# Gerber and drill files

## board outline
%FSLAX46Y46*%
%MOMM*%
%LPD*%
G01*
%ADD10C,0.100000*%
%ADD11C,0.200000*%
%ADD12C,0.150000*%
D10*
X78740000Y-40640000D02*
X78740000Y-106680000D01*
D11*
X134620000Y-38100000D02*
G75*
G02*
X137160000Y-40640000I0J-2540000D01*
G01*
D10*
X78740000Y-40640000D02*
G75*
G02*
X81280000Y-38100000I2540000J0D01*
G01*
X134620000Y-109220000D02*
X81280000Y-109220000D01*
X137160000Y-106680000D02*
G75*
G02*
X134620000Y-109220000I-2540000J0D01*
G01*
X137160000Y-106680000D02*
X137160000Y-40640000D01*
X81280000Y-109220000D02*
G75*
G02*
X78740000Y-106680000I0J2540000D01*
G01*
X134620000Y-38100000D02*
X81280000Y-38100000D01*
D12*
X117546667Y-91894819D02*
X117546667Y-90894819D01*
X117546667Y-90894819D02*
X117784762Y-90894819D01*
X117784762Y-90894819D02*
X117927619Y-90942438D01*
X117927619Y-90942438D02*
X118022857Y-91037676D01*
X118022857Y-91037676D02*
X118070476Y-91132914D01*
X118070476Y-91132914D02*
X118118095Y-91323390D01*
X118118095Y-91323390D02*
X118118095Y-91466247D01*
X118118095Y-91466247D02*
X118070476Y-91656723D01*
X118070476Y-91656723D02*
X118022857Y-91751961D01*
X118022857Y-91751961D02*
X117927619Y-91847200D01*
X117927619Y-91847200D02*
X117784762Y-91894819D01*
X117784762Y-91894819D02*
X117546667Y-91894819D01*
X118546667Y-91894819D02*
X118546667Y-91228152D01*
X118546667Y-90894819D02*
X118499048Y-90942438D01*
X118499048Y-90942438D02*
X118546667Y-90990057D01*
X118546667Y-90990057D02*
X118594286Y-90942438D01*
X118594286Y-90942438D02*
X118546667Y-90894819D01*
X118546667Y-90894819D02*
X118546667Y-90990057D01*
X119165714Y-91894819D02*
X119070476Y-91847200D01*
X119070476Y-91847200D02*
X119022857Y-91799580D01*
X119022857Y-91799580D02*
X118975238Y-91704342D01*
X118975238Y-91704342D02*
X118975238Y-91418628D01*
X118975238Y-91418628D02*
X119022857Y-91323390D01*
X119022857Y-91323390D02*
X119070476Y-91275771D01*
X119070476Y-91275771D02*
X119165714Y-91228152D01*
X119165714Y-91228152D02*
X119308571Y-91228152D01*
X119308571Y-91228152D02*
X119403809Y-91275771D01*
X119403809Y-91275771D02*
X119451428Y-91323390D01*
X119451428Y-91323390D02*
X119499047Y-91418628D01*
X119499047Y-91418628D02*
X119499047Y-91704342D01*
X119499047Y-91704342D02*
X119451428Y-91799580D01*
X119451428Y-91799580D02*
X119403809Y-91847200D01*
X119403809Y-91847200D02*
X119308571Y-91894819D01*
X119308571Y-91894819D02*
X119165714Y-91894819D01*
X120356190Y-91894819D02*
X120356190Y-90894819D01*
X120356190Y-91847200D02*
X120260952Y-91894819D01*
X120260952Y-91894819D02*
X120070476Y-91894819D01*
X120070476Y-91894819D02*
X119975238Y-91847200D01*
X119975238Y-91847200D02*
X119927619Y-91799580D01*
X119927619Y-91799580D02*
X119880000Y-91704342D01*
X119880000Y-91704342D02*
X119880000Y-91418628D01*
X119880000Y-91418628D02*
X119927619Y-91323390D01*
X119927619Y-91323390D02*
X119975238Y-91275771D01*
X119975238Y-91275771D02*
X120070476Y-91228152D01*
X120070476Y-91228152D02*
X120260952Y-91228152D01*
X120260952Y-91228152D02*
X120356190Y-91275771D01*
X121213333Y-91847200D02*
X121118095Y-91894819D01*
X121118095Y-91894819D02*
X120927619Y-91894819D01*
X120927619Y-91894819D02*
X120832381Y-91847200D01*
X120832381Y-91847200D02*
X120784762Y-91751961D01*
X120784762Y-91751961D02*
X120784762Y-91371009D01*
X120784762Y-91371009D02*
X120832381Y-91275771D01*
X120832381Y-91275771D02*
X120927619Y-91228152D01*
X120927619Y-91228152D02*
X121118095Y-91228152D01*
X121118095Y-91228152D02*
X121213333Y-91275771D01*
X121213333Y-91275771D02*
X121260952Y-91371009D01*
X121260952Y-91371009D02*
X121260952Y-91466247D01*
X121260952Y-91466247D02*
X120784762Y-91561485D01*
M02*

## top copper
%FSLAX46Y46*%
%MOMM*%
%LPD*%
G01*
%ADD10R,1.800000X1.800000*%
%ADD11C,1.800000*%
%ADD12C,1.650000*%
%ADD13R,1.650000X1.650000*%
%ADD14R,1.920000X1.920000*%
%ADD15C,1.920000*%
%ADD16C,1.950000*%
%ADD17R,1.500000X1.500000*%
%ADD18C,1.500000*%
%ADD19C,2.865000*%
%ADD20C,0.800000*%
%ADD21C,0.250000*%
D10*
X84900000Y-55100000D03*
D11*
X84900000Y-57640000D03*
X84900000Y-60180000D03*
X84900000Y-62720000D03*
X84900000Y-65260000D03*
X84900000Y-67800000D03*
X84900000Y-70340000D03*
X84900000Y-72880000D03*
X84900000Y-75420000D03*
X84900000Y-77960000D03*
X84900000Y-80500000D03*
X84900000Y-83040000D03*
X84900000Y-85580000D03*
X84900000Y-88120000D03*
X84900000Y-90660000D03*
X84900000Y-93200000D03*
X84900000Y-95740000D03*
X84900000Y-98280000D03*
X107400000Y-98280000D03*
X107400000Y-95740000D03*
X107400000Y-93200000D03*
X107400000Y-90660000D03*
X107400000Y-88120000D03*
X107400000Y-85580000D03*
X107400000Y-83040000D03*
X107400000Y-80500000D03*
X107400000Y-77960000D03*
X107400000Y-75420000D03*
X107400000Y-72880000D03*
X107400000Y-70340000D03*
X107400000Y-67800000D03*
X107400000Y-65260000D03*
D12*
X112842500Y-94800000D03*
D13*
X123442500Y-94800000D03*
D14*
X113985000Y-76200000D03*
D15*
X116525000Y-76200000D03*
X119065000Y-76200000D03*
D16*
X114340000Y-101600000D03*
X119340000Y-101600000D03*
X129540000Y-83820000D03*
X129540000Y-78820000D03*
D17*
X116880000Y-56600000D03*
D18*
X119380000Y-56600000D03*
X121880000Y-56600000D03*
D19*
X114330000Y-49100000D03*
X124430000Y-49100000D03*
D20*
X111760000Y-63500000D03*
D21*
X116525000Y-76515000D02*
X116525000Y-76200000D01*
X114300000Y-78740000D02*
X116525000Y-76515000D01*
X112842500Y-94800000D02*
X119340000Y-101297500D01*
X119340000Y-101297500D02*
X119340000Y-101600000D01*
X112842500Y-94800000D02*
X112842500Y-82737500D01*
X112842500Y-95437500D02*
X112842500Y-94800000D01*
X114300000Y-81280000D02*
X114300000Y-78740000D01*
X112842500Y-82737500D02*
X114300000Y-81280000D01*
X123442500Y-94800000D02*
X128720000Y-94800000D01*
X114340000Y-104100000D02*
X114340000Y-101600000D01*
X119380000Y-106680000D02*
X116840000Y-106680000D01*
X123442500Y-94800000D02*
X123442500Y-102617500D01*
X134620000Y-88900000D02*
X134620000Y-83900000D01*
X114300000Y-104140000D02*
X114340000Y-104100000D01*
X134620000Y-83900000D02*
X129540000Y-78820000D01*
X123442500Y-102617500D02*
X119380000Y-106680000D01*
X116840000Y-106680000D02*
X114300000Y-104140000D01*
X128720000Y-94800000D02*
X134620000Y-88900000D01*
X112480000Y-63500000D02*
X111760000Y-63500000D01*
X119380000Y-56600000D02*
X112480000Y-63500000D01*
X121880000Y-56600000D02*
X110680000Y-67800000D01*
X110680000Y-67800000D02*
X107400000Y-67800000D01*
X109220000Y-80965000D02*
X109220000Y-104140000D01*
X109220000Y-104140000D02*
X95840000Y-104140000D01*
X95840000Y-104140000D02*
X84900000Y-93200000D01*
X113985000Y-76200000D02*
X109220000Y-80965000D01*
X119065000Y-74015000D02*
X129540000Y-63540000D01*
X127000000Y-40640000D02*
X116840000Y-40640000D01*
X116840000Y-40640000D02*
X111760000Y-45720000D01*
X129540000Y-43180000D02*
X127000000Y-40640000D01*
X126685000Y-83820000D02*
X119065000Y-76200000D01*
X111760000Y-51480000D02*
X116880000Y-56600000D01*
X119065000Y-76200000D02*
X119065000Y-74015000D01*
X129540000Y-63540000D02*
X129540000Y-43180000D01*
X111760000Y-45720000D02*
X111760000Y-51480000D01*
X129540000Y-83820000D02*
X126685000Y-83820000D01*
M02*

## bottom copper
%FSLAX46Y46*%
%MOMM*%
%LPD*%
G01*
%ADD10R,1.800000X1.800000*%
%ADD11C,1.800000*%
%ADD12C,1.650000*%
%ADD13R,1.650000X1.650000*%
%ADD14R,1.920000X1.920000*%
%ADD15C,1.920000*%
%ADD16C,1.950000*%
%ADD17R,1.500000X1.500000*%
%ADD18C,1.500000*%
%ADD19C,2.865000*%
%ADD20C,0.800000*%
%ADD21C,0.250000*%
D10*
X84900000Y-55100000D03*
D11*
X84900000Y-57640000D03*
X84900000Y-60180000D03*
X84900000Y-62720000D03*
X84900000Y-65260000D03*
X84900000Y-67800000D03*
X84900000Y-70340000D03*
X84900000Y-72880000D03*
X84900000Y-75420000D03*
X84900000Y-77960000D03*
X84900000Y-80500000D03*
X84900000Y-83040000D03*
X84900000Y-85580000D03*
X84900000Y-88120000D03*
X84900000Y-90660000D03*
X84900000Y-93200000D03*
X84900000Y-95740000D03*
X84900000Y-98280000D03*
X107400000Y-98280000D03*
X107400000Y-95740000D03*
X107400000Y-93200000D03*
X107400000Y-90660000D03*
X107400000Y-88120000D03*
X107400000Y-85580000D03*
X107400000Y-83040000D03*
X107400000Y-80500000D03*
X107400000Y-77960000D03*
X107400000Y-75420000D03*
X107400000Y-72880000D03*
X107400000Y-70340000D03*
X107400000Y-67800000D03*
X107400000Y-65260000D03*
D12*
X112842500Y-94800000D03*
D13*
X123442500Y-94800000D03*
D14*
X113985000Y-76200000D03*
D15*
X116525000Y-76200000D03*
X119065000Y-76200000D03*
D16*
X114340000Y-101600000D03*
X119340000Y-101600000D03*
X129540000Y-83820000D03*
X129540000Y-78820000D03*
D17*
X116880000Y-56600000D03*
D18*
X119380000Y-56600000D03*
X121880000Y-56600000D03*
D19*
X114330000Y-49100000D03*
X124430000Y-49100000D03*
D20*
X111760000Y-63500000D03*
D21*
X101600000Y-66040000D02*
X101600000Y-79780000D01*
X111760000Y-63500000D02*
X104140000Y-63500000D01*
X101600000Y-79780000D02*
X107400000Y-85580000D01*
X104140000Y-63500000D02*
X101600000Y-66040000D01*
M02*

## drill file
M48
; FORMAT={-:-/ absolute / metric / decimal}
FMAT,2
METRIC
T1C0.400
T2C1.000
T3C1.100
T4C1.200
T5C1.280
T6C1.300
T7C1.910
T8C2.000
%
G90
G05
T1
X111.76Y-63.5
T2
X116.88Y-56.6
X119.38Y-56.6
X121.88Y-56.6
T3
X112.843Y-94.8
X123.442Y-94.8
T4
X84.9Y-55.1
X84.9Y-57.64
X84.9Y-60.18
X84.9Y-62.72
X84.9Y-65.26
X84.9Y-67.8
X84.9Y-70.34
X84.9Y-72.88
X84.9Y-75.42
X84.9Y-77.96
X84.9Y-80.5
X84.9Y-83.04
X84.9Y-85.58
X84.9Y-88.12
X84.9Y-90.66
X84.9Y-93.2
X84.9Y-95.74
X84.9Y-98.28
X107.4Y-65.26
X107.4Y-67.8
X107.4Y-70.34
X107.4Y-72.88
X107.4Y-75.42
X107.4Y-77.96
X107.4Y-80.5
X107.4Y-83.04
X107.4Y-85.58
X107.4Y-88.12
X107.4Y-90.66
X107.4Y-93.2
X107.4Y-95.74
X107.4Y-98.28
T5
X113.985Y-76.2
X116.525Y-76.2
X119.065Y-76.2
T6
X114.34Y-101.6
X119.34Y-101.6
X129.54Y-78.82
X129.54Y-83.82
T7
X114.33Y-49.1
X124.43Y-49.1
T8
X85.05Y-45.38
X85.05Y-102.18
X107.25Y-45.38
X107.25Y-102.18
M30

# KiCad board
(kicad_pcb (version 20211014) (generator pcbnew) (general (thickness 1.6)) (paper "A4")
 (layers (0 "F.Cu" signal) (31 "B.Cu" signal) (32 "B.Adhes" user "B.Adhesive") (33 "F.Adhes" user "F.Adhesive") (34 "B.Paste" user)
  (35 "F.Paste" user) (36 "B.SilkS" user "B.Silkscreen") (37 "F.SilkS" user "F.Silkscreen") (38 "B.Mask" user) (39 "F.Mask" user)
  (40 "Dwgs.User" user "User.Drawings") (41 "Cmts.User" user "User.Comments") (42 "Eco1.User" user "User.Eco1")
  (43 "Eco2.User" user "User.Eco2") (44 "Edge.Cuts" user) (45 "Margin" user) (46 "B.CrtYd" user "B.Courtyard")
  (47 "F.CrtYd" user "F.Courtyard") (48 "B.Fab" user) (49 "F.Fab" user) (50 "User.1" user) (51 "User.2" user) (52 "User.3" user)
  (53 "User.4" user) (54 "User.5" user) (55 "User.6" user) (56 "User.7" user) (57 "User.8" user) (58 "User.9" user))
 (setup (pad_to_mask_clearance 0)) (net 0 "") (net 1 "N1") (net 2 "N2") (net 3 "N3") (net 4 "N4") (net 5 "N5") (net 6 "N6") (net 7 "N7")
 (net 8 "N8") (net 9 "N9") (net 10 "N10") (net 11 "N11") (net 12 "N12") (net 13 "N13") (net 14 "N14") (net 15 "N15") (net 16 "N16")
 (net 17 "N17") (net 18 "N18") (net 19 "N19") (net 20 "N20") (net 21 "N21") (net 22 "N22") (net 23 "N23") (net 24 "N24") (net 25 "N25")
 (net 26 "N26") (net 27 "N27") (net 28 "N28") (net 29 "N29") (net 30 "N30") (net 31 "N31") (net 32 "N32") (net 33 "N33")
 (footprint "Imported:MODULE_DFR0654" (layer "F.Cu") (at 96.15 73.78)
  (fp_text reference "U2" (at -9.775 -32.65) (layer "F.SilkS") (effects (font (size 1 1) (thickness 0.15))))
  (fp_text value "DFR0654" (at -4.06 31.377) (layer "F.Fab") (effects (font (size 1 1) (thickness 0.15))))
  (pad "" np_thru_hole circle (at 11.1 28.4) (size 2 2) (drill 2) (layers *.Cu *.Mask))
  (pad "" np_thru_hole circle (at 11.1 -28.4) (size 2 2) (drill 2) (layers *.Cu *.Mask))
  (pad "" np_thru_hole circle (at -11.1 -28.4) (size 2 2) (drill 2) (layers *.Cu *.Mask))
  (pad "" np_thru_hole circle (at -11.1 28.4) (size 2 2) (drill 2) (layers *.Cu *.Mask))
  (pad "1" thru_hole rect (at -11.25 -18.68) (size 1.8 1.8) (drill 1.2) (layers *.Cu *.Mask) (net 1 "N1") (solder_mask_margin 0.102))
  (pad "2" thru_hole circle (at -11.25 -16.14) (size 1.8 1.8) (drill 1.2) (layers *.Cu *.Mask) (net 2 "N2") (solder_mask_margin 0.102))
  (pad "3" thru_hole circle (at -11.25 -13.6) (size 1.8 1.8) (drill 1.2) (layers *.Cu *.Mask) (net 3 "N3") (solder_mask_margin 0.102))
  (pad "4" thru_hole circle (at -11.25 -11.06) (size 1.8 1.8) (drill 1.2) (layers *.Cu *.Mask) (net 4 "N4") (solder_mask_margin 0.102))
  (pad "5" thru_hole circle (at -11.25 -8.52) (size 1.8 1.8) (drill 1.2) (layers *.Cu *.Mask) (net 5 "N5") (solder_mask_margin 0.102))
  (pad "6" thru_hole circle (at -11.25 -5.98) (size 1.8 1.8) (drill 1.2) (layers *.Cu *.Mask) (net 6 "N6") (solder_mask_margin 0.102))
  (pad "7" thru_hole circle (at -11.25 -3.44) (size 1.8 1.8) (drill 1.2) (layers *.Cu *.Mask) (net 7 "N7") (solder_mask_margin 0.102))
  (pad "8" thru_hole circle (at -11.25 -0.9) (size 1.8 1.8) (drill 1.2) (layers *.Cu *.Mask) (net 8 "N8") (solder_mask_margin 0.102))
  (pad "9" thru_hole circle (at -11.25 1.64) (size 1.8 1.8) (drill 1.2) (layers *.Cu *.Mask) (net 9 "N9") (solder_mask_margin 0.102))
  (pad "10" thru_hole circle (at -11.25 4.18) (size 1.8 1.8) (drill 1.2) (layers *.Cu *.Mask) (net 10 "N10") (solder_mask_margin 0.102))
  (pad "11" thru_hole circle (at -11.25 6.72) (size 1.8 1.8) (drill 1.2) (layers *.Cu *.Mask) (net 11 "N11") (solder_mask_margin 0.102))
  (pad "12" thru_hole circle (at -11.25 9.26) (size 1.8 1.8) (drill 1.2) (layers *.Cu *.Mask) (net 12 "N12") (solder_mask_margin 0.102))
  (pad "13" thru_hole circle (at -11.25 11.8) (size 1.8 1.8) (drill 1.2) (layers *.Cu *.Mask) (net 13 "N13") (solder_mask_margin 0.102))
  (pad "14" thru_hole circle (at -11.25 14.34) (size 1.8 1.8) (drill 1.2) (layers *.Cu *.Mask) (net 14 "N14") (solder_mask_margin 0.102))
  (pad "15" thru_hole circle (at -11.25 16.88) (size 1.8 1.8) (drill 1.2) (layers *.Cu *.Mask) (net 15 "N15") (solder_mask_margin 0.102))
  (pad "16" thru_hole circle (at -11.25 19.42) (size 1.8 1.8) (drill 1.2) (layers *.Cu *.Mask) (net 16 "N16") (solder_mask_margin 0.102))
  (pad "17" thru_hole circle (at -11.25 21.96) (size 1.8 1.8) (drill 1.2) (layers *.Cu *.Mask) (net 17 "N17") (solder_mask_margin 0.102))
  (pad "18" thru_hole circle (at -11.25 24.5) (size 1.8 1.8) (drill 1.2) (layers *.Cu *.Mask) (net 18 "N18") (solder_mask_margin 0.102))
  (pad "19" thru_hole circle (at 11.25 24.5) (size 1.8 1.8) (drill 1.2) (layers *.Cu *.Mask) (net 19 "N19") (solder_mask_margin 0.102))
  (pad "20" thru_hole circle (at 11.25 21.96) (size 1.8 1.8) (drill 1.2) (layers *.Cu *.Mask) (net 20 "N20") (solder_mask_margin 0.102))
  (pad "21" thru_hole circle (at 11.25 19.42) (size 1.8 1.8) (drill 1.2) (layers *.Cu *.Mask) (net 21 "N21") (solder_mask_margin 0.102))
  (pad "22" thru_hole circle (at 11.25 16.88) (size 1.8 1.8) (drill 1.2) (layers *.Cu *.Mask) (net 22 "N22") (solder_mask_margin 0.102))
  (pad "23" thru_hole circle (at 11.25 14.34) (size 1.8 1.8) (drill 1.2) (layers *.Cu *.Mask) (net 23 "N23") (solder_mask_margin 0.102))
  (pad "24" thru_hole circle (at 11.25 11.8) (size 1.8 1.8) (drill 1.2) (layers *.Cu *.Mask) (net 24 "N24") (solder_mask_margin 0.102))
  (pad "25" thru_hole circle (at 11.25 9.26) (size 1.8 1.8) (drill 1.2) (layers *.Cu *.Mask) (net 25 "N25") (solder_mask_margin 0.102))
  (pad "26" thru_hole circle (at 11.25 6.72) (size 1.8 1.8) (drill 1.2) (layers *.Cu *.Mask) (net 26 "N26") (solder_mask_margin 0.102))
  (pad "27" thru_hole circle (at 11.25 4.18) (size 1.8 1.8) (drill 1.2) (layers *.Cu *.Mask) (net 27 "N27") (solder_mask_margin 0.102))
  (pad "28" thru_hole circle (at 11.25 1.64) (size 1.8 1.8) (drill 1.2) (layers *.Cu *.Mask) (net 10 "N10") (solder_mask_margin 0.102))
  (pad "29" thru_hole circle (at 11.25 -0.9) (size 1.8 1.8) (drill 1.2) (layers *.Cu *.Mask) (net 9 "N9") (solder_mask_margin 0.102))
  (pad "30" thru_hole circle (at 11.25 -3.44) (size 1.8 1.8) (drill 1.2) (layers *.Cu *.Mask) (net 4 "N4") (solder_mask_margin 0.102))
  (pad "31" thru_hole circle (at 11.25 -5.98) (size 1.8 1.8) (drill 1.2) (layers *.Cu *.Mask) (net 2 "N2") (solder_mask_margin 0.102))
  (pad "32" thru_hole circle (at 11.25 -8.52) (size 1.8 1.8) (drill 1.2) (layers *.Cu *.Mask) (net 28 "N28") (solder_mask_margin 0.102)))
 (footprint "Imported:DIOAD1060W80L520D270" (layer "F.Cu") (at 118.1425 94.8 180)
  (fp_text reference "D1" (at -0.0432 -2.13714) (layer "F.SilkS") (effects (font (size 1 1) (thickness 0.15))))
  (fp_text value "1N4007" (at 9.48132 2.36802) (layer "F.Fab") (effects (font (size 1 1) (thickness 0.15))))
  (pad "A" thru_hole circle (at 5.3 0 180) (size 1.65 1.65) (drill 1.1) (layers *.Cu *.Mask) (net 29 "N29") (solder_mask_margin 0.102))
  (pad "C" thru_hole rect (at -5.3 0 180) (size 1.65 1.65) (drill 1.1) (layers *.Cu *.Mask) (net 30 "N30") (solder_mask_margin 0.102)))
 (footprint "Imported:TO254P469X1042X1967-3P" (layer "F.Cu") (at 113.985 76.2)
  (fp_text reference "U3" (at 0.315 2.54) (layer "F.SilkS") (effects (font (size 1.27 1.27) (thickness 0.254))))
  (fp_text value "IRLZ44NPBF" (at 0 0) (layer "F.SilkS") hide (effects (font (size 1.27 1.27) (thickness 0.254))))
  (pad "1" thru_hole rect (at 0 0) (size 1.92 1.92) (drill 1.28) (layers *.Cu *.Mask) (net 16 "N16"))
  (pad "2" thru_hole circle (at 2.54 0) (size 1.92 1.92) (drill 1.28) (layers *.Cu *.Mask) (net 29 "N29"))
  (pad "3" thru_hole circle (at 5.08 0) (size 1.92 1.92) (drill 1.28) (layers *.Cu *.Mask) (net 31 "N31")))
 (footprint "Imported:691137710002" (layer "F.Cu") (at 116.84 101.6)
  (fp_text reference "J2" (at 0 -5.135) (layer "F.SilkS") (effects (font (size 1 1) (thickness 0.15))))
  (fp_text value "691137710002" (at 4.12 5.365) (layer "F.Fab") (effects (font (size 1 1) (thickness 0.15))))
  (pad "1" thru_hole circle (at -2.5 0) (size 1.95 1.95) (drill 1.3) (layers *.Cu *.Mask) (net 30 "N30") (solder_mask_margin 0.102))
  (pad "2" thru_hole circle (at 2.5 0) (size 1.95 1.95) (drill 1.3) (layers *.Cu *.Mask) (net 29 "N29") (solder_mask_margin 0.102)))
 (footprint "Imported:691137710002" (layer "F.Cu") (at 129.54 81.32 90)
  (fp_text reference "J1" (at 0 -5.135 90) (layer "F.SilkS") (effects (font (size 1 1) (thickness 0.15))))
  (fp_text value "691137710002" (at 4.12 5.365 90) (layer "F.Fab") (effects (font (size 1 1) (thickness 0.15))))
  (pad "1" thru_hole circle (at -2.5 0 90) (size 1.95 1.95) (drill 1.3) (layers *.Cu *.Mask) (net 31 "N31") (solder_mask_margin 0.102))
  (pad "2" thru_hole circle (at 2.5 0 90) (size 1.95 1.95) (drill 1.3) (layers *.Cu *.Mask) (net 30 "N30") (solder_mask_margin 0.102)))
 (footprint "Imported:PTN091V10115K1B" (layer "F.Cu") (at 116.88 56.6)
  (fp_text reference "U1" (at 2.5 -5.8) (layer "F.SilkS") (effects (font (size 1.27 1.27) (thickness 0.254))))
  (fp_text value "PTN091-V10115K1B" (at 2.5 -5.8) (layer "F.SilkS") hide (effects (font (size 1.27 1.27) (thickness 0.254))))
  (pad "1" thru_hole rect (at 0 0) (size 1.5 1.5) (drill 1) (layers *.Cu *.Mask) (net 31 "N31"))
  (pad "2" thru_hole circle (at 2.5 0) (size 1.5 1.5) (drill 1) (layers *.Cu *.Mask) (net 24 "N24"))
  (pad "3" thru_hole circle (at 5 0) (size 1.5 1.5) (drill 1) (layers *.Cu *.Mask) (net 2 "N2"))
  (pad "4" thru_hole circle (at -2.55 -7.5) (size 2.865 2.865) (drill 1.91) (layers *.Cu *.Mask) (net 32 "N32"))
  (pad "5" thru_hole circle (at 7.55 -7.5) (size 2.865 2.865) (drill 1.91) (layers *.Cu *.Mask) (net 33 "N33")))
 (gr_line (start 78.74 40.64) (end 78.74 106.68) (layer "Edge.Cuts") (width 0.1))
 (gr_arc (start 134.62 38.1) (mid 136.416051 38.843949) (end 137.16 40.64) (layer "Edge.Cuts") (width 0.2))
 (gr_arc (start 78.74 40.64) (mid 79.483949 38.843949) (end 81.28 38.1) (layer "Edge.Cuts") (width 0.1))
 (gr_line (start 134.62 109.22) (end 81.28 109.22) (layer "Edge.Cuts") (width 0.1))
 (gr_arc (start 137.16 106.68) (mid 136.416051 108.476051) (end 134.62 109.22) (layer "Edge.Cuts") (width 0.1))
 (gr_line (start 137.16 106.68) (end 137.16 40.64) (layer "Edge.Cuts") (width 0.1))
 (gr_arc (start 81.28 109.22) (mid 79.483949 108.476051) (end 78.74 106.68) (layer "Edge.Cuts") (width 0.1))
 (gr_line (start 134.62 38.1) (end 81.28 38.1) (layer "Edge.Cuts") (width 0.1))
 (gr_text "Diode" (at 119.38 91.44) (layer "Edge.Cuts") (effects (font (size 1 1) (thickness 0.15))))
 (segment (start 116.525 76.515) (end 116.525 76.2) (width 0.25) (layer "F.Cu") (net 29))
 (segment (start 114.3 78.74) (end 116.525 76.515) (width 0.25) (layer "F.Cu") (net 29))
 (segment (start 112.8425 94.8) (end 119.34 101.2975) (width 0.25) (layer "F.Cu") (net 29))
 (segment (start 119.34 101.2975) (end 119.34 101.6) (width 0.25) (layer "F.Cu") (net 29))
 (segment (start 112.8425 94.8) (end 112.8425 82.7375) (width 0.25) (layer "F.Cu") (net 29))
 (segment (start 112.8425 95.4375) (end 112.8425 94.8) (width 0.25) (layer "F.Cu") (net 29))
 (segment (start 114.3 81.28) (end 114.3 78.74) (width 0.25) (layer "F.Cu") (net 29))
 (segment (start 112.8425 82.7375) (end 114.3 81.28) (width 0.25) (layer "F.Cu") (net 29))
 (segment (start 123.4425 94.8) (end 128.72 94.8) (width 0.25) (layer "F.Cu") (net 30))
 (segment (start 114.34 104.1) (end 114.34 101.6) (width 0.25) (layer "F.Cu") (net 30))
 (segment (start 119.38 106.68) (end 116.84 106.68) (width 0.25) (layer "F.Cu") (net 30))
 (segment (start 123.4425 94.8) (end 123.4425 102.6175) (width 0.25) (layer "F.Cu") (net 30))
 (segment (start 134.62 88.9) (end 134.62 83.9) (width 0.25) (layer "F.Cu") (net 30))
 (segment (start 114.3 104.14) (end 114.34 104.1) (width 0.25) (layer "F.Cu") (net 30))
 (segment (start 134.62 83.9) (end 129.54 78.82) (width 0.25) (layer "F.Cu") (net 30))
 (segment (start 123.4425 102.6175) (end 119.38 106.68) (width 0.25) (layer "F.Cu") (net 30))
 (segment (start 116.84 106.68) (end 114.3 104.14) (width 0.25) (layer "F.Cu") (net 30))
 (segment (start 128.72 94.8) (end 134.62 88.9) (width 0.25) (layer "F.Cu") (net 30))
 (segment (start 112.48 63.5) (end 111.76 63.5) (width 0.25) (layer "F.Cu") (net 24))
 (segment (start 119.38 56.6) (end 112.48 63.5) (width 0.25) (layer "F.Cu") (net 24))
 (via (at 111.76 63.5) (size 0.8) (drill 0.4) (layers "F.Cu" "B.Cu") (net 24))
 (segment (start 101.6 66.04) (end 101.6 79.78) (width 0.25) (layer "B.Cu") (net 24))
 (segment (start 111.76 63.5) (end 104.14 63.5) (width 0.25) (layer "B.Cu") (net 24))
 (segment (start 101.6 79.78) (end 107.4 85.58) (width 0.25) (layer "B.Cu") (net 24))
 (segment (start 104.14 63.5) (end 101.6 66.04) (width 0.25) (layer "B.Cu") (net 24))
 (segment (start 121.88 56.6) (end 110.68 67.8) (width 0.25) (layer "F.Cu") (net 2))
 (segment (start 110.68 67.8) (end 107.4 67.8) (width 0.25) (layer "F.Cu") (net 2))
 (segment (start 109.22 80.965) (end 109.22 104.14) (width 0.25) (layer "F.Cu") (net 16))
 (segment (start 109.22 104.14) (end 95.84 104.14) (width 0.25) (layer "F.Cu") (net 16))
 (segment (start 95.84 104.14) (end 84.9 93.2) (width 0.25) (layer "F.Cu") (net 16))
 (segment (start 113.985 76.2) (end 109.22 80.965) (width 0.25) (layer "F.Cu") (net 16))
 (segment (start 119.065 74.015) (end 129.54 63.54) (width 0.25) (layer "F.Cu") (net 31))
 (segment (start 127 40.64) (end 116.84 40.64) (width 0.25) (layer "F.Cu") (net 31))
 (segment (start 116.84 40.64) (end 111.76 45.72) (width 0.25) (layer "F.Cu") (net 31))
 (segment (start 129.54 43.18) (end 127 40.64) (width 0.25) (layer "F.Cu") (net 31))
 (segment (start 126.685 83.82) (end 119.065 76.2) (width 0.25) (layer "F.Cu") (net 31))
 (segment (start 111.76 51.48) (end 116.88 56.6) (width 0.25) (layer "F.Cu") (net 31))
 (segment (start 119.065 76.2) (end 119.065 74.015) (width 0.25) (layer "F.Cu") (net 31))
 (segment (start 129.54 63.54) (end 129.54 43.18) (width 0.25) (layer "F.Cu") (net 31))
 (segment (start 111.76 45.72) (end 111.76 51.48) (width 0.25) (layer "F.Cu") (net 31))
 (segment (start 129.54 83.82) (end 126.685 83.82) (width 0.25) (layer "F.Cu") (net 31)))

